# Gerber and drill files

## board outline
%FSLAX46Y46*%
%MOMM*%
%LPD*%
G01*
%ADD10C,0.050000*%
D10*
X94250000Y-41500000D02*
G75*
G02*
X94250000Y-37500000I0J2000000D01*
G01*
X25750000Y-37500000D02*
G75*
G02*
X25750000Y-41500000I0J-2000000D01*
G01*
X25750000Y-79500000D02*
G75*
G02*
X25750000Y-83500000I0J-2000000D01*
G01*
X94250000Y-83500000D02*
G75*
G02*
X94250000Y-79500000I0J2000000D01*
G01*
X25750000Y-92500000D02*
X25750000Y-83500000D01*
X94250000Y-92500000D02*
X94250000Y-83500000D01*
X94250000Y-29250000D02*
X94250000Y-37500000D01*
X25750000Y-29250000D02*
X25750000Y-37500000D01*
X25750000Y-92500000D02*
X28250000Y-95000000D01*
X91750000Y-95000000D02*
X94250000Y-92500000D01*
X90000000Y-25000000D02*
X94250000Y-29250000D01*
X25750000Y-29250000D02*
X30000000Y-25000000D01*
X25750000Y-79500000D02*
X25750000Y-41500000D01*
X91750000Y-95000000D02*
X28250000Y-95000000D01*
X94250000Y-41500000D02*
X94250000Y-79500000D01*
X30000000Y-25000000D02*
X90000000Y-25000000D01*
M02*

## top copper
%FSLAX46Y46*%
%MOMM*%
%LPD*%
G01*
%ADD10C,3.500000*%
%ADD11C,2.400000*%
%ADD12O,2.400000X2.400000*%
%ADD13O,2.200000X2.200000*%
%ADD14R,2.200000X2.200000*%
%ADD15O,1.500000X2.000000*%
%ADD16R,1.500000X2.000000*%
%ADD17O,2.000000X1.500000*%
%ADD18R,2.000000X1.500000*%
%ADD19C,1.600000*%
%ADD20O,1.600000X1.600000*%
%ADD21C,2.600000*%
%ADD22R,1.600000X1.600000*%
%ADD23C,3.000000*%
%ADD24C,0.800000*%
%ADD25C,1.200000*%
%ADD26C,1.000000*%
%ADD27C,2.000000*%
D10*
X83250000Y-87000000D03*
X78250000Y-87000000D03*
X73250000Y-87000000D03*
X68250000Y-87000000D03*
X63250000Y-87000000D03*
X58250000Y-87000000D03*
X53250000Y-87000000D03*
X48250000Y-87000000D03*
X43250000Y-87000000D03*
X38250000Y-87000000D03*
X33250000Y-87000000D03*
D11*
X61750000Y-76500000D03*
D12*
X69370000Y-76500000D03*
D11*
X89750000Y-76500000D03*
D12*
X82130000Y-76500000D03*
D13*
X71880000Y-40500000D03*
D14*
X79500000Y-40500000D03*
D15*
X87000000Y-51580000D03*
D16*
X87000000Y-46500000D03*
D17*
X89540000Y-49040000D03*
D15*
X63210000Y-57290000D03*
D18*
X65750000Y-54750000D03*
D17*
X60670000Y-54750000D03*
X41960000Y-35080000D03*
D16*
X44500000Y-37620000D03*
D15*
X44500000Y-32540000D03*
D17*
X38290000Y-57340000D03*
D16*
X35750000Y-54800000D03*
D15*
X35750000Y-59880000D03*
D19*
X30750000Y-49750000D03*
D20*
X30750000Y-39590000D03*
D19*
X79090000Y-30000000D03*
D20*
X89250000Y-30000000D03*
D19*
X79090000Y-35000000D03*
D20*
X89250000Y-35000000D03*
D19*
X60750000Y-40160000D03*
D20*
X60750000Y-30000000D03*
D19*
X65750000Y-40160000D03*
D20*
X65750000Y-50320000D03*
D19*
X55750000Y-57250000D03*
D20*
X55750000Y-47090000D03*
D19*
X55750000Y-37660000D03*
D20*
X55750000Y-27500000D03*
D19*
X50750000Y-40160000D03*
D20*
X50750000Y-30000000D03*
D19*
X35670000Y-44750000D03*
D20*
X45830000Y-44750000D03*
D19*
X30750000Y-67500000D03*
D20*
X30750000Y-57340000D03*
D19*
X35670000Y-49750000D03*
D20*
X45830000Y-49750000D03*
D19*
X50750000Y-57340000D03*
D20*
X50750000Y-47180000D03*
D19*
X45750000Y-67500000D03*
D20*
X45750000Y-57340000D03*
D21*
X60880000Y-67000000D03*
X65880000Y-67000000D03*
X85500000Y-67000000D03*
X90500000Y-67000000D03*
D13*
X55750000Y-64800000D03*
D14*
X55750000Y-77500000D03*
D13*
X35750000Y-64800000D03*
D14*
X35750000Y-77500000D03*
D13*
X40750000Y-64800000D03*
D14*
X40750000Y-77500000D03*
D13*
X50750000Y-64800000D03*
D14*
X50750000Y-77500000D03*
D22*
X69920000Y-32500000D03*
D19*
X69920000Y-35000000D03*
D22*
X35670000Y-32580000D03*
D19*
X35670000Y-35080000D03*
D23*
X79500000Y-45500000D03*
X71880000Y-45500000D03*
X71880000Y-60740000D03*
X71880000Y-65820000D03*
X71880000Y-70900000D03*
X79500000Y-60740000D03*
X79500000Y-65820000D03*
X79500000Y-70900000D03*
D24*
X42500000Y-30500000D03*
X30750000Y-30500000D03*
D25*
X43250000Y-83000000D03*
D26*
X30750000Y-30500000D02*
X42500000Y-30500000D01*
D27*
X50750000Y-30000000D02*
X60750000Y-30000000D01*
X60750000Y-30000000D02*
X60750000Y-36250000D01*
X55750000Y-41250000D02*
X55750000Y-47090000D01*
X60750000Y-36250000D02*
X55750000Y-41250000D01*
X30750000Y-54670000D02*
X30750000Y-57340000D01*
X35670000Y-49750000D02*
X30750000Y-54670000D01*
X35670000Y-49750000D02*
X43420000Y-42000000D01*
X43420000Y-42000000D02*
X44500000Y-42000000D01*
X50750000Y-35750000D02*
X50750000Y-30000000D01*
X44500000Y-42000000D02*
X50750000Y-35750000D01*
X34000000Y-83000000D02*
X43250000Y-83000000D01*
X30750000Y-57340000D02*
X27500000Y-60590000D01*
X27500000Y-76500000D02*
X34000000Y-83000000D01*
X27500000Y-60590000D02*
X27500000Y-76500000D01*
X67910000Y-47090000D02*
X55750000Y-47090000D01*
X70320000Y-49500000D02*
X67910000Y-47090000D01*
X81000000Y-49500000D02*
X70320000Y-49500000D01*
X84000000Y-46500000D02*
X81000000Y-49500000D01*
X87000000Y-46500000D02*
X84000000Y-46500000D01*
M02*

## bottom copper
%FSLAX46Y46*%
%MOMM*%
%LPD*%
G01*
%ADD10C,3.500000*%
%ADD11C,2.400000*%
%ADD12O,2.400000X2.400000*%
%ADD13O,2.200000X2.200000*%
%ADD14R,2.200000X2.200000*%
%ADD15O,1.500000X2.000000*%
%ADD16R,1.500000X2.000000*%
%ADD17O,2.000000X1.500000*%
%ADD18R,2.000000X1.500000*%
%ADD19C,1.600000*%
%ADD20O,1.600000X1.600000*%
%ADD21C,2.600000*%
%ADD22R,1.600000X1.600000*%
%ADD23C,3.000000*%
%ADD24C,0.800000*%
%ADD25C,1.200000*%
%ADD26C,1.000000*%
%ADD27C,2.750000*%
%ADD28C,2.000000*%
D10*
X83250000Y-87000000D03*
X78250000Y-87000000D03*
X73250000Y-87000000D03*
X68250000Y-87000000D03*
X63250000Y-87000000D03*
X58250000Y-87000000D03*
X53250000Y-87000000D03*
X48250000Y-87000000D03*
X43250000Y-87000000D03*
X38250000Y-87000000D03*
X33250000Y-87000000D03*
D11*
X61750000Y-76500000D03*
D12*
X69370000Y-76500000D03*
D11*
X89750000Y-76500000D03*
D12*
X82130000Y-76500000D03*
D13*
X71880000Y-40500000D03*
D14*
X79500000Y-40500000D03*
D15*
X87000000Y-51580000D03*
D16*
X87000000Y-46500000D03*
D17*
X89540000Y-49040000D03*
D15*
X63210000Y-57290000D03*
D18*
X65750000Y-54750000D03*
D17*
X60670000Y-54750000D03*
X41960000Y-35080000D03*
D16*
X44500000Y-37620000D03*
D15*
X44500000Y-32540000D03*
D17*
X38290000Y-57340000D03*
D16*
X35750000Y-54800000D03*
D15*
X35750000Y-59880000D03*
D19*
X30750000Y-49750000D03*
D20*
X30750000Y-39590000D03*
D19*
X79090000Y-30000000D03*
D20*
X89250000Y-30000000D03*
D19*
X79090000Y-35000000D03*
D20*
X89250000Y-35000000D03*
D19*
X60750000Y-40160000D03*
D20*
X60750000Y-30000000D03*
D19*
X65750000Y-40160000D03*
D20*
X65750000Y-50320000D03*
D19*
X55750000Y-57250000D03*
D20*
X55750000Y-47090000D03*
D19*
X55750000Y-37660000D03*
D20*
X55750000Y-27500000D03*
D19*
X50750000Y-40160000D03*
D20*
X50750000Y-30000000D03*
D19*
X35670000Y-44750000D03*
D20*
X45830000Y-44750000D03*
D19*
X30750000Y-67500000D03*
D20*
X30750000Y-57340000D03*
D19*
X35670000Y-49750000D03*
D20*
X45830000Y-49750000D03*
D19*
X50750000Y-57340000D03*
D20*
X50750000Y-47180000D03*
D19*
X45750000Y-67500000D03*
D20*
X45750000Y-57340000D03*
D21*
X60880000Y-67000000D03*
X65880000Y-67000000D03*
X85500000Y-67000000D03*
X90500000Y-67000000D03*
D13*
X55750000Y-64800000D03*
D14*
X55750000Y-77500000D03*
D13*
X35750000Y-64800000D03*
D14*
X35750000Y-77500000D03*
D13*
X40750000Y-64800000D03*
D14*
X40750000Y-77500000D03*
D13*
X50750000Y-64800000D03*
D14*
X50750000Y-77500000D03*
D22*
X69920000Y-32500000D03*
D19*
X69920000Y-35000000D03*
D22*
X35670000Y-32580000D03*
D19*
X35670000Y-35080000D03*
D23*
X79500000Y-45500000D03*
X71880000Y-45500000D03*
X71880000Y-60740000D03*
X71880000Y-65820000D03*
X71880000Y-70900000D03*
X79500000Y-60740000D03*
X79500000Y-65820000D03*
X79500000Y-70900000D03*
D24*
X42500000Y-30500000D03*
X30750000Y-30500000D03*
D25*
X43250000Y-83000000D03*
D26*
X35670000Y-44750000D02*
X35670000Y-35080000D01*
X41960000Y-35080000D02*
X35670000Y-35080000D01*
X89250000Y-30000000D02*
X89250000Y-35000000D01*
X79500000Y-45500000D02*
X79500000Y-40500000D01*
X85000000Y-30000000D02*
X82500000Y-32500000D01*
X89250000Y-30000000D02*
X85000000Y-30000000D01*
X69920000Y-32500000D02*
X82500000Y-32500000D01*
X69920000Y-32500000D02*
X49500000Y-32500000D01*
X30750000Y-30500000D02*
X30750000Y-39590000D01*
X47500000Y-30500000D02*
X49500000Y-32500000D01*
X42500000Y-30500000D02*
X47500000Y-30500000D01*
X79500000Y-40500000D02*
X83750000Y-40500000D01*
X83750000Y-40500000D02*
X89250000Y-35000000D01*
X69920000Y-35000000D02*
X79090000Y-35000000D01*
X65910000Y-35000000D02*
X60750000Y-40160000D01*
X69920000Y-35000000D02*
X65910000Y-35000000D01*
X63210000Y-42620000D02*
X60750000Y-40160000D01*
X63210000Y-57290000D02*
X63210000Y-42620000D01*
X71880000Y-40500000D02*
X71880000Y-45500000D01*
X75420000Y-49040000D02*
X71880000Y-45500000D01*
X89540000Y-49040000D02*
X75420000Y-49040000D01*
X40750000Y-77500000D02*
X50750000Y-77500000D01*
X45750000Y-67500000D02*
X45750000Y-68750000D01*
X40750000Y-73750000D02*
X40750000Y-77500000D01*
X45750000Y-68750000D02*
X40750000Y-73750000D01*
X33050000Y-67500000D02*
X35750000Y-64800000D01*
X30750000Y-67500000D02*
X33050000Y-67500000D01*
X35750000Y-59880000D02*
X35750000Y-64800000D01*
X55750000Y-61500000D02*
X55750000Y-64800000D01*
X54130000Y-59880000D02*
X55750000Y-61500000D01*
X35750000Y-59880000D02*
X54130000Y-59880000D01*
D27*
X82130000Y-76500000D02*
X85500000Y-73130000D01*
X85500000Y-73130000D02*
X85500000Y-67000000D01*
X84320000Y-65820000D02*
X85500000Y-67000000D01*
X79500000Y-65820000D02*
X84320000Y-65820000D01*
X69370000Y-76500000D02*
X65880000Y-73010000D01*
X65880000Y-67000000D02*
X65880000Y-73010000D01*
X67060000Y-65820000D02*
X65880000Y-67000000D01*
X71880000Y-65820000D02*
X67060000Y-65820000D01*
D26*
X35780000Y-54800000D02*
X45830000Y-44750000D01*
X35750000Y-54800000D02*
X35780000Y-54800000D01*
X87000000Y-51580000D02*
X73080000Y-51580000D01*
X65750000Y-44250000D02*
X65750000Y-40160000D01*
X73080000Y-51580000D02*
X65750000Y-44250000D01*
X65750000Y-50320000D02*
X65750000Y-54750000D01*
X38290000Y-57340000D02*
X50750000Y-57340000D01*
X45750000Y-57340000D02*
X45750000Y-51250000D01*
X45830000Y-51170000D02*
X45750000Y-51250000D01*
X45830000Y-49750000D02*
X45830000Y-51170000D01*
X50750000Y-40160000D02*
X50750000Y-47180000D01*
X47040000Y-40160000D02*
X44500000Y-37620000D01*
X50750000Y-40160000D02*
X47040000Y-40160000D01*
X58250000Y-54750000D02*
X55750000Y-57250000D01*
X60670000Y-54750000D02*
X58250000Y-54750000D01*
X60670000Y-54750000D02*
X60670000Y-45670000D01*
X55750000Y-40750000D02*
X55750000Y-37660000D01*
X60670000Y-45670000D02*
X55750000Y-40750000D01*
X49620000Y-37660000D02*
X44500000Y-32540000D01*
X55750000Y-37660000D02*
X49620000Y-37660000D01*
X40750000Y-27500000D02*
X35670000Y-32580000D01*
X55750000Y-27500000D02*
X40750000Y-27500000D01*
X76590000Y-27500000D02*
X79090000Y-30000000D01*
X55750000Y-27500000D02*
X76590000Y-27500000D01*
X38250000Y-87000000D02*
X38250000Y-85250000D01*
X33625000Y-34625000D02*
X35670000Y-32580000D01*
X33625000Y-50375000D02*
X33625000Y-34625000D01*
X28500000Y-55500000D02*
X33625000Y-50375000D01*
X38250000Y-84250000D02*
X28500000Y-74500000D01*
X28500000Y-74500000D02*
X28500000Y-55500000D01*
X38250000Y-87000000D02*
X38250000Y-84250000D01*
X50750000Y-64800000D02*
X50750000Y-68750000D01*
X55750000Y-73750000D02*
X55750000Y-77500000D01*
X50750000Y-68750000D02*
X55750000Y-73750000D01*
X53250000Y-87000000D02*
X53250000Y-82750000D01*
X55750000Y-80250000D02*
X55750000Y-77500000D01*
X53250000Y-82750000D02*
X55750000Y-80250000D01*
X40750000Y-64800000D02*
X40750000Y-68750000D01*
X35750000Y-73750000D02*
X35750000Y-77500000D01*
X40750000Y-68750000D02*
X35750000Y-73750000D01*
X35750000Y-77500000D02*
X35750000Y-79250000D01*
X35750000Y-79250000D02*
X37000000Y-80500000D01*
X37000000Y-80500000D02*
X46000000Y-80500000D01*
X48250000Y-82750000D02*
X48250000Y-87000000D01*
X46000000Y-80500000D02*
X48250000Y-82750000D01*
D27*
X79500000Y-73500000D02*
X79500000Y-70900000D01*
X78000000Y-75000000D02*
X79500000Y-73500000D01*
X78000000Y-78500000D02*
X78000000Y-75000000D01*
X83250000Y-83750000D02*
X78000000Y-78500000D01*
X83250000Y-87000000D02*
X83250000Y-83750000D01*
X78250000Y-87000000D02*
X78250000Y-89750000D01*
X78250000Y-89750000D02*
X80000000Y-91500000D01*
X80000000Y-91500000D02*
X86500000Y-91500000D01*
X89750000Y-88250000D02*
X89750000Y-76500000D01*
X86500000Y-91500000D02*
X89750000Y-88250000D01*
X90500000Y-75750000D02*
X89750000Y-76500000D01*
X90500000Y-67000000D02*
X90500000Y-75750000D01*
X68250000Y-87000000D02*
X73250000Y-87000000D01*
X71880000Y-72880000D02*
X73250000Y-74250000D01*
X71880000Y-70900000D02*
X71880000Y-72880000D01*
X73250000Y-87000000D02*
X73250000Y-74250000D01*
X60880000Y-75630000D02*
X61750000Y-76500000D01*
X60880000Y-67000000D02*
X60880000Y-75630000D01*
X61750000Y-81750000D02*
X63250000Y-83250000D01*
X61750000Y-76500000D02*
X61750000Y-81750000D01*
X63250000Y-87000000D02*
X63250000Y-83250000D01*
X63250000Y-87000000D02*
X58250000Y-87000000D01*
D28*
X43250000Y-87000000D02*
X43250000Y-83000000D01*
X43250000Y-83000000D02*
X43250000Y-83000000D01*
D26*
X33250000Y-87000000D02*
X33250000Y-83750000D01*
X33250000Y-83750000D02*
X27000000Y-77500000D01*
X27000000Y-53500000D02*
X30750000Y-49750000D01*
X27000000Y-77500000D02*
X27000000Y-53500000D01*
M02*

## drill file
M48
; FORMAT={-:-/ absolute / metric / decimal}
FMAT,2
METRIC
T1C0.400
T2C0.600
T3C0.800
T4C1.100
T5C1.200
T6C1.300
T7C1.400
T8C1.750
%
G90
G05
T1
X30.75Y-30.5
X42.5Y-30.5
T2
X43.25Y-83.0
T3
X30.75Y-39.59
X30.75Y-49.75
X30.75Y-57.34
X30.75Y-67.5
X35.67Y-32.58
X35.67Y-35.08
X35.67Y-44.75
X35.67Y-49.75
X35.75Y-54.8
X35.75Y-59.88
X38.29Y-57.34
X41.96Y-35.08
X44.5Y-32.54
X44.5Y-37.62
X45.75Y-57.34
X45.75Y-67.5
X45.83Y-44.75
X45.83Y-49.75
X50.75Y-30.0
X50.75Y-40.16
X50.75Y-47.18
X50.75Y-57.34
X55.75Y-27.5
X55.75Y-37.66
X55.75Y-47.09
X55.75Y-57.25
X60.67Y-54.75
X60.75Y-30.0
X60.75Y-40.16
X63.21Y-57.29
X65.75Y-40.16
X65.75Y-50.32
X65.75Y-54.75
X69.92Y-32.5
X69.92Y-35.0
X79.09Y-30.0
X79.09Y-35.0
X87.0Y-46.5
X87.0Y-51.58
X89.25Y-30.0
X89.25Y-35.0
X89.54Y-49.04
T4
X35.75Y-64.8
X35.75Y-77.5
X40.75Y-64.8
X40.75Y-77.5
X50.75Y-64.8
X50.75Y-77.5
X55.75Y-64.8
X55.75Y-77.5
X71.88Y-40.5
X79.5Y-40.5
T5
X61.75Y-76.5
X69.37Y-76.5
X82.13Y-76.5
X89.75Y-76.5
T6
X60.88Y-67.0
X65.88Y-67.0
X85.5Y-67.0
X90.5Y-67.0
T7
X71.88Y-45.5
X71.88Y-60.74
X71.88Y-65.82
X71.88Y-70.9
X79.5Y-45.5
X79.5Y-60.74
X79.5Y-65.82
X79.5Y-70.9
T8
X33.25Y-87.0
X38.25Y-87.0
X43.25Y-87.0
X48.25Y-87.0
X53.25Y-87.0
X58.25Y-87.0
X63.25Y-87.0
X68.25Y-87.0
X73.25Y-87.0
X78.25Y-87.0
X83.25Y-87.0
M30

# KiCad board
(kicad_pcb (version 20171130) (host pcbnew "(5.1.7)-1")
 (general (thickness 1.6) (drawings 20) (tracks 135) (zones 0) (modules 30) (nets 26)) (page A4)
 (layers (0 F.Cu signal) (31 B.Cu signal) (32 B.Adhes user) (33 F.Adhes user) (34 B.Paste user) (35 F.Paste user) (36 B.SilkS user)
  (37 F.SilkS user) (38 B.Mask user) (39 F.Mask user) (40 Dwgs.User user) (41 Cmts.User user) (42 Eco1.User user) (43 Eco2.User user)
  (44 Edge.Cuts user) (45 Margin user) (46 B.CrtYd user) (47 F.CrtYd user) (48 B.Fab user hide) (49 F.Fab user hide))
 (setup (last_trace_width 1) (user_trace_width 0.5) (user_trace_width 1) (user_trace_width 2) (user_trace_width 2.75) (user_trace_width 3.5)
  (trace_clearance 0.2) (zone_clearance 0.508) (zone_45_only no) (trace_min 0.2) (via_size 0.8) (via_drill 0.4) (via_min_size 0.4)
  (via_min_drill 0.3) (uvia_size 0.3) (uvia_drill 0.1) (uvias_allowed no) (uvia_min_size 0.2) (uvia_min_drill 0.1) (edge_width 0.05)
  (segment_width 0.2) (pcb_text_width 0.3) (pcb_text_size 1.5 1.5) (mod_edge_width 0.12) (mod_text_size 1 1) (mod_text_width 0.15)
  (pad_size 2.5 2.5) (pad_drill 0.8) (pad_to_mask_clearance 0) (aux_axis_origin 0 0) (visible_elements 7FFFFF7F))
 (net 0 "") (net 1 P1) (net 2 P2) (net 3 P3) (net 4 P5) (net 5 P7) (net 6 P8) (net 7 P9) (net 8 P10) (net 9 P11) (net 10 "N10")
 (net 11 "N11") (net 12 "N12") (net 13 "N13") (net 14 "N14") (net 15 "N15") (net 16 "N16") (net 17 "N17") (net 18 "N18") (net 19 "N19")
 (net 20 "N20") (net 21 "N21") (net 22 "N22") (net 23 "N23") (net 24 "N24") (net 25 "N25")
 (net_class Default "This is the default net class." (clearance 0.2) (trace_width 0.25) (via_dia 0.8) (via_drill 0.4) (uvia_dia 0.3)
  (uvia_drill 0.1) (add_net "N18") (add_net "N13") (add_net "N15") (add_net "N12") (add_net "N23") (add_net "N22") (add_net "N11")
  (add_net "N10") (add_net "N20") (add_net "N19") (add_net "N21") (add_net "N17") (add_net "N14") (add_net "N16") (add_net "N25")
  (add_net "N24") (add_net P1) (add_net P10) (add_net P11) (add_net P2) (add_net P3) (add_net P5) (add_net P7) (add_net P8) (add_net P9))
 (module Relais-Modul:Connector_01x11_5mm (layer F.Cu) (at 83.25 87)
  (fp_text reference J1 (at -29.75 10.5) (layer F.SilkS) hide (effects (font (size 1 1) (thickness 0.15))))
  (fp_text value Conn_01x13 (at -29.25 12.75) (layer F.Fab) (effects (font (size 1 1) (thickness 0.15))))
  (pad 1 thru_hole circle (at 0 0 180) (size 3.5 3.5) (drill 1.75) (layers B.Cu B.Mask) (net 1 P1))
  (pad 2 thru_hole circle (at -5 0 180) (size 3.5 3.5) (drill 1.75) (layers B.Cu B.Mask) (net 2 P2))
  (pad 3 thru_hole circle (at -10 0 180) (size 3.5 3.5) (drill 1.75) (layers B.Cu B.Mask) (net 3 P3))
  (pad 4 thru_hole circle (at -15 0 180) (size 3.5 3.5) (drill 1.75) (layers B.Cu B.Mask) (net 3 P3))
  (pad 5 thru_hole circle (at -20 0 180) (size 3.5 3.5) (drill 1.75) (layers B.Cu B.Mask) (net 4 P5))
  (pad 6 thru_hole circle (at -25 0 180) (size 3.5 3.5) (drill 1.75) (layers B.Cu B.Mask) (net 4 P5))
  (pad 7 thru_hole circle (at -30 0 180) (size 3.5 3.5) (drill 1.75) (layers B.Cu B.Mask) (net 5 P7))
  (pad 8 thru_hole circle (at -35 0 180) (size 3.5 3.5) (drill 1.75) (layers B.Cu B.Mask) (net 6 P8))
  (pad 9 thru_hole circle (at -40 0 180) (size 3.5 3.5) (drill 1.75) (layers B.Cu B.Mask) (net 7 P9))
  (pad 10 thru_hole circle (at -45 0 180) (size 3.5 3.5) (drill 1.75) (layers B.Cu B.Mask) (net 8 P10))
  (pad 11 thru_hole circle (at -50 0 180) (size 3.5 3.5) (drill 1.75) (layers B.Cu B.Mask) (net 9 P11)))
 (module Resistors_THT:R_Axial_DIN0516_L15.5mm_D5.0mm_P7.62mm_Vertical (layer F.Cu) (at 61.75 76.5)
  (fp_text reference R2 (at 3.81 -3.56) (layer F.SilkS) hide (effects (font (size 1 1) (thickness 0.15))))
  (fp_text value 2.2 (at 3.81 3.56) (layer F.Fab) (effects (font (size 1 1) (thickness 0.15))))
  (pad 1 thru_hole circle (at 0 0) (size 2.4 2.4) (drill 1.2) (layers *.Cu *.Mask) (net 4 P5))
  (pad 2 thru_hole oval (at 7.62 0) (size 2.4 2.4) (drill 1.2) (layers *.Cu *.Mask) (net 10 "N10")))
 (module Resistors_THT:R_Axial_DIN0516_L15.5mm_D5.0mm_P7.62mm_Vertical (layer F.Cu) (at 89.75 76.5 180)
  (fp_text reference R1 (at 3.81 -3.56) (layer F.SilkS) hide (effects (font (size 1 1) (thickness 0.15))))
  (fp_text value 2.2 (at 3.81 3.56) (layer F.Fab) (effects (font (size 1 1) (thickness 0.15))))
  (pad 1 thru_hole circle (at 0 0 180) (size 2.4 2.4) (drill 1.2) (layers *.Cu *.Mask) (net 2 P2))
  (pad 2 thru_hole oval (at 7.62 0 180) (size 2.4 2.4) (drill 1.2) (layers *.Cu *.Mask) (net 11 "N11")))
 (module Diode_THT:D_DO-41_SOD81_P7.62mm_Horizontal (layer F.Cu) (at 79.5 40.5 180)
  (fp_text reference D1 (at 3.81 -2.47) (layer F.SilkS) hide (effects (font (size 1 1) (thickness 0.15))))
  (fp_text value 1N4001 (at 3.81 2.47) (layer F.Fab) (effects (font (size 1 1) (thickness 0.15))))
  (pad 2 thru_hole oval (at 7.62 0 180) (size 2.2 2.2) (drill 1.1) (layers *.Cu *.Mask) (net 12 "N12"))
  (pad 1 thru_hole rect (at 0 0 180) (size 2.2 2.2) (drill 1.1) (layers *.Cu *.Mask) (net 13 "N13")))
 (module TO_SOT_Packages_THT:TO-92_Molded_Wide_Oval (layer F.Cu) (at 87 46.5 270)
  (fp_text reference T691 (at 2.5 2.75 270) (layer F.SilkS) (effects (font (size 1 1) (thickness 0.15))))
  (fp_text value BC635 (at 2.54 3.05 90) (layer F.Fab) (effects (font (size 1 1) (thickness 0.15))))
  (pad 3 thru_hole oval (at 5.08 0) (size 1.5 2) (drill 0.8) (layers *.Cu *.Mask) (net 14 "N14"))
  (pad 1 thru_hole rect (at 0 0) (size 1.5 2) (drill 0.8) (layers *.Cu *.Mask) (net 7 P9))
  (pad 2 thru_hole oval (at 2.54 -2.54) (size 2 1.5) (drill 0.8) (layers *.Cu *.Mask) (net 12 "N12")))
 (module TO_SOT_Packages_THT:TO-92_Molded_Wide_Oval (layer F.Cu) (at 65.75 54.75 180)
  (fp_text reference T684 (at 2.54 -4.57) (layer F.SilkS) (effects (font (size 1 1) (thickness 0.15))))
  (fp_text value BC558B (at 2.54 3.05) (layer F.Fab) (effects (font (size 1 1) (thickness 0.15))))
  (pad 2 thru_hole oval (at 2.54 -2.54 270) (size 2 1.5) (drill 0.8) (layers *.Cu *.Mask) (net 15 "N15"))
  (pad 1 thru_hole rect (at 0 0 270) (size 1.5 2) (drill 0.8) (layers *.Cu *.Mask) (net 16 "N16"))
  (pad 3 thru_hole oval (at 5.08 0 270) (size 1.5 2) (drill 0.8) (layers *.Cu *.Mask) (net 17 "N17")))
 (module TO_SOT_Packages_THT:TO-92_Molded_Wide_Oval (layer F.Cu) (at 44.5 37.62 90)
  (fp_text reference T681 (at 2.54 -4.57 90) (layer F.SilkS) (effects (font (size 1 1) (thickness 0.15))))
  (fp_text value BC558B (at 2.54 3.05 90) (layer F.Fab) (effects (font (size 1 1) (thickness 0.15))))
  (pad 2 thru_hole oval (at 2.54 -2.54 180) (size 2 1.5) (drill 0.8) (layers *.Cu *.Mask) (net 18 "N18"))
  (pad 1 thru_hole rect (at 0 0 180) (size 1.5 2) (drill 0.8) (layers *.Cu *.Mask) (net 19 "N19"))
  (pad 3 thru_hole oval (at 5.08 0 180) (size 1.5 2) (drill 0.8) (layers *.Cu *.Mask) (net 17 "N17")))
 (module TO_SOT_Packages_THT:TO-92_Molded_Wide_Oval (layer F.Cu) (at 35.75 54.8 270)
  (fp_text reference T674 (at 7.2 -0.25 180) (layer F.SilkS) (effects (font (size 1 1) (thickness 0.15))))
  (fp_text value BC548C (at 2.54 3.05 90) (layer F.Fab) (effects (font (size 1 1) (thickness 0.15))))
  (pad 2 thru_hole oval (at 2.54 -2.54) (size 2 1.5) (drill 0.8) (layers *.Cu *.Mask) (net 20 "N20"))
  (pad 1 thru_hole rect (at 0 0) (size 1.5 2) (drill 0.8) (layers *.Cu *.Mask) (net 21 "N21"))
  (pad 3 thru_hole oval (at 5.08 0) (size 1.5 2) (drill 0.8) (layers *.Cu *.Mask) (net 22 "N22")))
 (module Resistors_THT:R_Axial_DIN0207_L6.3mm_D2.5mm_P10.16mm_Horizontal (layer F.Cu) (at 30.75 49.75 90)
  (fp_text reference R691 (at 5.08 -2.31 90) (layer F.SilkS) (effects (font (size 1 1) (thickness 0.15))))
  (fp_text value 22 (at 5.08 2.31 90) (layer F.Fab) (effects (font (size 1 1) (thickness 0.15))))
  (pad 1 thru_hole circle (at 0 0 90) (size 1.6 1.6) (drill 0.8) (layers *.Cu *.Mask) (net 9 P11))
  (pad 2 thru_hole oval (at 10.16 0 90) (size 1.6 1.6) (drill 0.8) (layers *.Cu *.Mask) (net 13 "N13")))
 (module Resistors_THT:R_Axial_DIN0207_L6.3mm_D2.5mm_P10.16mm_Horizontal (layer F.Cu) (at 79.09 30)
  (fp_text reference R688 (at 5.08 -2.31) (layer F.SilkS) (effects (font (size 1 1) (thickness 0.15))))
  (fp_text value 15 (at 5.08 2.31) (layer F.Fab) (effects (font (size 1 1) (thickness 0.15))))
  (pad 1 thru_hole circle (at 0 0) (size 1.6 1.6) (drill 0.8) (layers *.Cu *.Mask) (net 8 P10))
  (pad 2 thru_hole oval (at 10.16 0) (size 1.6 1.6) (drill 0.8) (layers *.Cu *.Mask) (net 13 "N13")))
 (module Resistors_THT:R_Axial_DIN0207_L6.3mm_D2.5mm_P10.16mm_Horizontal (layer F.Cu) (at 79.09 35)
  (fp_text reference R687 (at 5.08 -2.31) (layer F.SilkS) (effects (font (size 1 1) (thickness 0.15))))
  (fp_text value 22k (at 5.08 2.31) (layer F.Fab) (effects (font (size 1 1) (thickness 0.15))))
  (pad 1 thru_hole circle (at 0 0) (size 1.6 1.6) (drill 0.8) (layers *.Cu *.Mask) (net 15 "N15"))
  (pad 2 thru_hole oval (at 10.16 0) (size 1.6 1.6) (drill 0.8) (layers *.Cu *.Mask) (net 13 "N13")))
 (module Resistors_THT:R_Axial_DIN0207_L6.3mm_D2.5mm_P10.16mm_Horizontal (layer F.Cu) (at 60.75 40.16 90)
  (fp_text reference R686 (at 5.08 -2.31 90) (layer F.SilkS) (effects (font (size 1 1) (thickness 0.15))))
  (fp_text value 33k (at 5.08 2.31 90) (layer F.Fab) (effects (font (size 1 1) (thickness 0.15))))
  (pad 1 thru_hole circle (at 0 0 90) (size 1.6 1.6) (drill 0.8) (layers *.Cu *.Mask) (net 15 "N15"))
  (pad 2 thru_hole oval (at 10.16 0 90) (size 1.6 1.6) (drill 0.8) (layers *.Cu *.Mask) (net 7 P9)))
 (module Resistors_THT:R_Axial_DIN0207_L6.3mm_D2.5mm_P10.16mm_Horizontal (layer F.Cu) (at 65.75 40.16 270)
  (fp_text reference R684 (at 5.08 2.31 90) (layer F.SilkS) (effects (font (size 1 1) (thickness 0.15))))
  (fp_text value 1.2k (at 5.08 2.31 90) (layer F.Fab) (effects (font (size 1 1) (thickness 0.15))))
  (pad 1 thru_hole circle (at 0 0 270) (size 1.6 1.6) (drill 0.8) (layers *.Cu *.Mask) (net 14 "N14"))
  (pad 2 thru_hole oval (at 10.16 0 270) (size 1.6 1.6) (drill 0.8) (layers *.Cu *.Mask) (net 16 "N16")))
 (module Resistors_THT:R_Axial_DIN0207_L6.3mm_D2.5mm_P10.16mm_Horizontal (layer F.Cu) (at 55.75 57.25 90)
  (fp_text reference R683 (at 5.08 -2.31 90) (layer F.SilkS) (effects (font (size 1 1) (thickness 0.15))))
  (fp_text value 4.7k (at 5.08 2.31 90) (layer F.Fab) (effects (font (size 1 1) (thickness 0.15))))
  (pad 1 thru_hole circle (at 0 0 90) (size 1.6 1.6) (drill 0.8) (layers *.Cu *.Mask) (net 17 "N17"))
  (pad 2 thru_hole oval (at 10.16 0 90) (size 1.6 1.6) (drill 0.8) (layers *.Cu *.Mask) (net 7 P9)))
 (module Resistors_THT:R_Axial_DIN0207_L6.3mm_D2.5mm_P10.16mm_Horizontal (layer F.Cu) (at 55.75 37.66 90)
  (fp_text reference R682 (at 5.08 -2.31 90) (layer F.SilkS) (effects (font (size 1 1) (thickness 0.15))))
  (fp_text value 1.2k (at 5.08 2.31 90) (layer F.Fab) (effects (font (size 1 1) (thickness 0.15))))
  (pad 1 thru_hole circle (at 0 0 90) (size 1.6 1.6) (drill 0.8) (layers *.Cu *.Mask) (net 17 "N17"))
  (pad 2 thru_hole oval (at 10.16 0 90) (size 1.6 1.6) (drill 0.8) (layers *.Cu *.Mask) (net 8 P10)))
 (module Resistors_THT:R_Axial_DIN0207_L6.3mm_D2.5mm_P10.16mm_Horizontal (layer F.Cu) (at 50.75 40.16 90)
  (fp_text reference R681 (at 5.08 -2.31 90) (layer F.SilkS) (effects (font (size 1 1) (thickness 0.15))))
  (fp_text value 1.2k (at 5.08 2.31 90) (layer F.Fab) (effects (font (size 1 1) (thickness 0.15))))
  (pad 1 thru_hole circle (at 0 0 90) (size 1.6 1.6) (drill 0.8) (layers *.Cu *.Mask) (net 19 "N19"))
  (pad 2 thru_hole oval (at 10.16 0 90) (size 1.6 1.6) (drill 0.8) (layers *.Cu *.Mask) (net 7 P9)))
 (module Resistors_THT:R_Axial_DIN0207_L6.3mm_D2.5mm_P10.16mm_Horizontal (layer F.Cu) (at 35.67 44.75)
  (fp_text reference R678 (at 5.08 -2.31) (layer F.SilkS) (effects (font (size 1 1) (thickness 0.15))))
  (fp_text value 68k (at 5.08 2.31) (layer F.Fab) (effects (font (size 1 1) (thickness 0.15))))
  (pad 1 thru_hole circle (at 0 0) (size 1.6 1.6) (drill 0.8) (layers *.Cu *.Mask) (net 18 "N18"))
  (pad 2 thru_hole oval (at 10.16 0) (size 1.6 1.6) (drill 0.8) (layers *.Cu *.Mask) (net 21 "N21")))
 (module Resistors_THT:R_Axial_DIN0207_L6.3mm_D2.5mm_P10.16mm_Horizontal (layer F.Cu) (at 30.75 67.5 90)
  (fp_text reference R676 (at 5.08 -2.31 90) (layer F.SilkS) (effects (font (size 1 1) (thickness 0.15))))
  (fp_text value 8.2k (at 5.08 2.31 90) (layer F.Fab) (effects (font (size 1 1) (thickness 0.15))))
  (pad 1 thru_hole circle (at 0 0 90) (size 1.6 1.6) (drill 0.8) (layers *.Cu *.Mask) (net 22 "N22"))
  (pad 2 thru_hole oval (at 10.16 0 90) (size 1.6 1.6) (drill 0.8) (layers *.Cu *.Mask) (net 7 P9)))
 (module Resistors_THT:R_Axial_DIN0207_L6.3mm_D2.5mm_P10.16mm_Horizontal (layer F.Cu) (at 35.67 49.75)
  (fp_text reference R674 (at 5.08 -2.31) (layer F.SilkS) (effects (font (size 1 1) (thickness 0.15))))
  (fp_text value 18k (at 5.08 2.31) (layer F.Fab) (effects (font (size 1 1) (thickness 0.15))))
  (pad 1 thru_hole circle (at 0 0) (size 1.6 1.6) (drill 0.8) (layers *.Cu *.Mask) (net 7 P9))
  (pad 2 thru_hole oval (at 10.16 0) (size 1.6 1.6) (drill 0.8) (layers *.Cu *.Mask) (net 20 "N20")))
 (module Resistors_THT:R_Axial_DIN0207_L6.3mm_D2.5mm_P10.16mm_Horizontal (layer F.Cu) (at 50.75 57.34 90)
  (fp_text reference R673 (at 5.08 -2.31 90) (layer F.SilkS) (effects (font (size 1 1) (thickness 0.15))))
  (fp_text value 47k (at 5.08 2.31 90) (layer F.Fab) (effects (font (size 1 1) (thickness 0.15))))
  (pad 1 thru_hole circle (at 0 0 90) (size 1.6 1.6) (drill 0.8) (layers *.Cu *.Mask) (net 20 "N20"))
  (pad 2 thru_hole oval (at 10.16 0 90) (size 1.6 1.6) (drill 0.8) (layers *.Cu *.Mask) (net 19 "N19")))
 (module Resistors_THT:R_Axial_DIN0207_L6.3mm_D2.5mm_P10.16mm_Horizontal (layer F.Cu) (at 45.75 67.5 90)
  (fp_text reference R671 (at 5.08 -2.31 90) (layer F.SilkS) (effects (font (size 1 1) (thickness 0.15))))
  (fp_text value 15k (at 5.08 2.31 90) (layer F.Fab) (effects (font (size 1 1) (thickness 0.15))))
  (pad 1 thru_hole circle (at 0 0 90) (size 1.6 1.6) (drill 0.8) (layers *.Cu *.Mask) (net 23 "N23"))
  (pad 2 thru_hole oval (at 10.16 0 90) (size 1.6 1.6) (drill 0.8) (layers *.Cu *.Mask) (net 20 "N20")))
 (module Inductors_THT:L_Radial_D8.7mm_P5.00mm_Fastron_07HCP (layer F.Cu) (at 60.88 67)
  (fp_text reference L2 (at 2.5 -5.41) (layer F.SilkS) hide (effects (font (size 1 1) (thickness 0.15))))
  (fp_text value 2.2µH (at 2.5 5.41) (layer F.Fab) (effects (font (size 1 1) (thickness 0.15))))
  (pad 1 thru_hole circle (at 0 0) (size 2.6 2.6) (drill 1.3) (layers *.Cu *.Mask) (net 4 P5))
  (pad 2 thru_hole circle (at 5 0) (size 2.6 2.6) (drill 1.3) (layers *.Cu *.Mask) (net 10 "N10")))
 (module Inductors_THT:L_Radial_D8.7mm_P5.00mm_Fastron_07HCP (layer F.Cu) (at 85.5 67)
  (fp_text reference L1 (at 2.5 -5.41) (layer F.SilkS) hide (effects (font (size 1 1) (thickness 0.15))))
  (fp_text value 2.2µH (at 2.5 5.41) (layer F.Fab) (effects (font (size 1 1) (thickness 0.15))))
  (pad 1 thru_hole circle (at 0 0) (size 2.6 2.6) (drill 1.3) (layers *.Cu *.Mask) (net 11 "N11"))
  (pad 2 thru_hole circle (at 5 0) (size 2.6 2.6) (drill 1.3) (layers *.Cu *.Mask) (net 2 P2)))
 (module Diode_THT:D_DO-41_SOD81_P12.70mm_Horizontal (layer F.Cu) (at 55.75 77.5 90)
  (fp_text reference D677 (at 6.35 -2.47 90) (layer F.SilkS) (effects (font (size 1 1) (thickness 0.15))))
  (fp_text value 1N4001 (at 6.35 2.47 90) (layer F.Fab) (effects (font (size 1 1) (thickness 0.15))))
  (pad 2 thru_hole oval (at 12.7 0 90) (size 2.2 2.2) (drill 1.1) (layers *.Cu *.Mask) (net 22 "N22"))
  (pad 1 thru_hole rect (at 0 0 90) (size 2.2 2.2) (drill 1.1) (layers *.Cu *.Mask) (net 5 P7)))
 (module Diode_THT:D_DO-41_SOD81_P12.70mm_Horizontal (layer F.Cu) (at 35.75 77.5 90)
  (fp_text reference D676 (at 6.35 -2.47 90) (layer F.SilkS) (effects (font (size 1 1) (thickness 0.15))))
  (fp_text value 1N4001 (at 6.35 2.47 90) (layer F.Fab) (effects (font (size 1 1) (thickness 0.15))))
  (pad 2 thru_hole oval (at 12.7 0 90) (size 2.2 2.2) (drill 1.1) (layers *.Cu *.Mask) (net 22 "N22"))
  (pad 1 thru_hole rect (at 0 0 90) (size 2.2 2.2) (drill 1.1) (layers *.Cu *.Mask) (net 6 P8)))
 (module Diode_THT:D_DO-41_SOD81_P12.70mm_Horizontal (layer F.Cu) (at 40.75 77.5 90)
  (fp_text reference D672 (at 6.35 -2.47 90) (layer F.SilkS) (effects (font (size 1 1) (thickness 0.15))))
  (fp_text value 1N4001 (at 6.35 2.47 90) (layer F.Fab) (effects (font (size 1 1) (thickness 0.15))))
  (pad 2 thru_hole oval (at 12.7 0 90) (size 2.2 2.2) (drill 1.1) (layers *.Cu *.Mask) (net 6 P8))
  (pad 1 thru_hole rect (at 0 0 90) (size 2.2 2.2) (drill 1.1) (layers *.Cu *.Mask) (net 23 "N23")))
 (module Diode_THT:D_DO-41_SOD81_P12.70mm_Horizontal (layer F.Cu) (at 50.75 77.5 90)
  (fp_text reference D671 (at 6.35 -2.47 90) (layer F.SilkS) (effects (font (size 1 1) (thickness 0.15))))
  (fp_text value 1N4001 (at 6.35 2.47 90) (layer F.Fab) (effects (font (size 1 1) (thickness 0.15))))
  (pad 2 thru_hole oval (at 12.7 0 90) (size 2.2 2.2) (drill 1.1) (layers *.Cu *.Mask) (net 5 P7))
  (pad 1 thru_hole rect (at 0 0 90) (size 2.2 2.2) (drill 1.1) (layers *.Cu *.Mask) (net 23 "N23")))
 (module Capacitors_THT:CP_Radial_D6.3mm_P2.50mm (layer F.Cu) (at 69.92 32.5 270)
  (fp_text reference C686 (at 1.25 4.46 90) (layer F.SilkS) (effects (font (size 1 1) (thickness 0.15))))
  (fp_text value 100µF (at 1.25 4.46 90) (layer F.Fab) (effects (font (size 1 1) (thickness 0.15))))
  (pad 1 thru_hole rect (at 0 0 270) (size 1.6 1.6) (drill 0.8) (layers *.Cu *.Mask) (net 13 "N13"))
  (pad 2 thru_hole circle (at 2.5 0 270) (size 1.6 1.6) (drill 0.8) (layers *.Cu *.Mask) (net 15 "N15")))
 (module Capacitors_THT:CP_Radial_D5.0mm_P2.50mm (layer F.Cu) (at 35.67 32.58 270)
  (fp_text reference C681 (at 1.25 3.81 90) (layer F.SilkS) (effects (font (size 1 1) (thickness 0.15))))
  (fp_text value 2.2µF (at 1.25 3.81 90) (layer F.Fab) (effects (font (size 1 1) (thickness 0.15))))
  (pad 1 thru_hole rect (at 0 0 270) (size 1.6 1.6) (drill 0.8) (layers *.Cu *.Mask) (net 8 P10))
  (pad 2 thru_hole circle (at 2.5 0 270) (size 1.6 1.6) (drill 0.8) (layers *.Cu *.Mask) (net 18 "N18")))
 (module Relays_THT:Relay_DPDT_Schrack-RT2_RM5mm (layer F.Cu) (at 79.5 45.5 270)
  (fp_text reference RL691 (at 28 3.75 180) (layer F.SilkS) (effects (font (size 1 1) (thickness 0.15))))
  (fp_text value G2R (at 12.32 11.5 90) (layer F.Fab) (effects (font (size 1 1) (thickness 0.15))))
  (pad A1 thru_hole circle (at 0 0 270) (size 3 3) (drill 1.4) (layers *.Cu *.Mask) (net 13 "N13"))
  (pad A2 thru_hole circle (at 0 7.62 270) (size 3 3) (drill 1.4) (layers *.Cu *.Mask) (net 12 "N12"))
  (pad 22 thru_hole circle (at 15.24 7.62 270) (size 3 3) (drill 1.4) (layers *.Cu *.Mask) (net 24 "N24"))
  (pad 21 thru_hole circle (at 20.32 7.62 270) (size 3 3) (drill 1.4) (layers *.Cu *.Mask) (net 10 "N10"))
  (pad 24 thru_hole circle (at 25.4 7.62 270) (size 3 3) (drill 1.4) (layers *.Cu *.Mask) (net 3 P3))
  (pad 12 thru_hole circle (at 15.24 0 270) (size 3 3) (drill 1.4) (layers *.Cu *.Mask) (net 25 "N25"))
  (pad 11 thru_hole circle (at 20.32 0 270) (size 3 3) (drill 1.4) (layers *.Cu *.Mask) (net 11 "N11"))
  (pad 14 thru_hole circle (at 25.4 0 270) (size 3 3) (drill 1.4) (layers *.Cu *.Mask) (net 1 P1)))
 (gr_arc (start 94.25 39.5) (end 94.25 37.5) (angle -180) (layer Edge.Cuts) (width 0.05))
 (gr_arc (start 25.75 39.5) (end 25.75 41.5) (angle -180) (layer Edge.Cuts) (width 0.05))
 (gr_arc (start 25.75 81.5) (end 25.75 83.5) (angle -180) (layer Edge.Cuts) (width 0.05))
 (gr_arc (start 94.25 81.5) (end 94.25 79.5) (angle -180) (layer Edge.Cuts) (width 0.05))
 (gr_line (start 25.75 92.5) (end 25.75 83.5) (layer Edge.Cuts) (width 0.05))
 (gr_line (start 94.25 92.5) (end 94.25 83.5) (layer Edge.Cuts) (width 0.05))
 (gr_line (start 94.25 29.25) (end 94.25 37.5) (layer Edge.Cuts) (width 0.05))
 (gr_line (start 25.75 29.25) (end 25.75 37.5) (layer Edge.Cuts) (width 0.05))
 (gr_line (start 25.75 92.5) (end 28.25 95) (layer Edge.Cuts) (width 0.05))
 (gr_line (start 91.75 95) (end 94.25 92.5) (layer Edge.Cuts) (width 0.05))
 (gr_line (start 90 25) (end 94.25 29.25) (layer Edge.Cuts) (width 0.05))
 (gr_line (start 25.75 29.25) (end 30 25) (layer Edge.Cuts) (width 0.05))
 (gr_line (start 25.75 79.5) (end 25.75 41.5) (layer Edge.Cuts) (width 0.05))
 (gr_line (start 91.75 95) (end 28.25 95) (layer Edge.Cuts) (width 0.05))
 (gr_line (start 94.25 41.5) (end 94.25 79.5) (layer Edge.Cuts) (width 0.05))
 (gr_line (start 30 25) (end 90 25) (layer Edge.Cuts) (width 0.05))
 (segment (start 35.67 44.75) (end 35.67 35.08) (width 1) (layer B.Cu) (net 18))
 (segment (start 41.96 35.08) (end 35.67 35.08) (width 1) (layer B.Cu) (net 18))
 (segment (start 89.25 30) (end 89.25 35) (width 1) (layer B.Cu) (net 13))
 (segment (start 79.5 45.5) (end 79.5 40.5) (width 1) (layer B.Cu) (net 13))
 (segment (start 85 30) (end 82.5 32.5) (width 1) (layer B.Cu) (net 13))
 (segment (start 89.25 30) (end 85 30) (width 1) (layer B.Cu) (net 13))
 (segment (start 69.92 32.5) (end 82.5 32.5) (width 1) (layer B.Cu) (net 13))
 (segment (start 69.92 32.5) (end 49.5 32.5) (width 1) (layer B.Cu) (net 13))
 (via (at 42.5 30.5) (size 0.8) (drill 0.4) (layers F.Cu B.Cu) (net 13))
 (via (at 30.75 30.5) (size 0.8) (drill 0.4) (layers F.Cu B.Cu) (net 13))
 (segment (start 30.75 30.5) (end 42.5 30.5) (width 1) (layer F.Cu) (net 13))
 (segment (start 30.75 30.5) (end 30.75 39.59) (width 1) (layer B.Cu) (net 13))
 (segment (start 47.5 30.5) (end 49.5 32.5) (width 1) (layer B.Cu) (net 13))
 (segment (start 42.5 30.5) (end 47.5 30.5) (width 1) (layer B.Cu) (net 13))
 (segment (start 79.5 40.5) (end 83.75 40.5) (width 1) (layer B.Cu) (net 13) (status 1000000))
 (segment (start 83.75 40.5) (end 89.25 35) (width 1) (layer B.Cu) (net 13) (status 1000000))
 (segment (start 69.92 35) (end 79.09 35) (width 1) (layer B.Cu) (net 15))
 (segment (start 65.91 35) (end 60.75 40.16) (width 1) (layer B.Cu) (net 15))
 (segment (start 69.92 35) (end 65.91 35) (width 1) (layer B.Cu) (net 15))
 (segment (start 63.21 42.62) (end 60.75 40.16) (width 1) (layer B.Cu) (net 15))
 (segment (start 63.21 57.29) (end 63.21 42.62) (width 1) (layer B.Cu) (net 15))
 (segment (start 71.88 40.5) (end 71.88 45.5) (width 1) (layer B.Cu) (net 12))
 (segment (start 75.42 49.04) (end 71.88 45.5) (width 1) (layer B.Cu) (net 12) (status 1000000))
 (segment (start 89.54 49.04) (end 75.42 49.04) (width 1) (layer B.Cu) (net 12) (status 1000000))
 (segment (start 40.75 77.5) (end 50.75 77.5) (width 1) (layer B.Cu) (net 23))
 (segment (start 45.75 67.5) (end 45.75 68.75) (width 1) (layer B.Cu) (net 23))
 (segment (start 40.75 73.75) (end 40.75 77.5) (width 1) (layer B.Cu) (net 23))
 (segment (start 45.75 68.75) (end 40.75 73.75) (width 1) (layer B.Cu) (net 23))
 (segment (start 33.05 67.5) (end 35.75 64.8) (width 1) (layer B.Cu) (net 22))
 (segment (start 30.75 67.5) (end 33.05 67.5) (width 1) (layer B.Cu) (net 22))
 (segment (start 35.75 59.88) (end 35.75 64.8) (width 1) (layer B.Cu) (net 22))
 (segment (start 55.75 61.5) (end 55.75 64.8) (width 1) (layer B.Cu) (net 22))
 (segment (start 54.13 59.88) (end 55.75 61.5) (width 1) (layer B.Cu) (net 22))
 (segment (start 35.75 59.88) (end 54.13 59.88) (width 1) (layer B.Cu) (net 22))
 (segment (start 82.13 76.5) (end 85.5 73.13) (width 2.75) (layer B.Cu) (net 11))
 (segment (start 85.5 73.13) (end 85.5 67) (width 2.75) (layer B.Cu) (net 11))
 (segment (start 84.32 65.82) (end 85.5 67) (width 2.75) (layer B.Cu) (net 11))
 (segment (start 79.5 65.82) (end 84.32 65.82) (width 2.75) (layer B.Cu) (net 11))
 (segment (start 69.37 76.5) (end 65.88 73.01) (width 2.75) (layer B.Cu) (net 10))
 (segment (start 65.88 67) (end 65.88 73.01) (width 2.75) (layer B.Cu) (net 10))
 (segment (start 67.06 65.82) (end 65.88 67) (width 2.75) (layer B.Cu) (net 10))
 (segment (start 71.88 65.82) (end 67.06 65.82) (width 2.75) (layer B.Cu) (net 10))
 (segment (start 35.78 54.8) (end 45.83 44.75) (width 1) (layer B.Cu) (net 21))
 (segment (start 35.75 54.8) (end 35.78 54.8) (width 1) (layer B.Cu) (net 21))
 (segment (start 87 51.58) (end 73.08 51.58) (width 1) (layer B.Cu) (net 14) (status 1000000))
 (segment (start 65.75 44.25) (end 65.75 40.16) (width 1) (layer B.Cu) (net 14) (status 1000000))
 (segment (start 73.08 51.58) (end 65.75 44.25) (width 1) (layer B.Cu) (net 14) (status 1000000))
 (segment (start 65.75 50.32) (end 65.75 54.75) (width 1) (layer B.Cu) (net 16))
 (segment (start 38.29 57.34) (end 50.75 57.34) (width 1) (layer B.Cu) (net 20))
 (segment (start 45.75 57.34) (end 45.75 51.25) (width 1) (layer B.Cu) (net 20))
 (segment (start 45.83 51.17) (end 45.75 51.25) (width 1) (layer B.Cu) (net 20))
 (segment (start 45.83 49.75) (end 45.83 51.17) (width 1) (layer B.Cu) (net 20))
 (segment (start 50.75 40.16) (end 50.75 47.18) (width 1) (layer B.Cu) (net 19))
 (segment (start 47.04 40.16) (end 44.5 37.62) (width 1) (layer B.Cu) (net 19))
 (segment (start 50.75 40.16) (end 47.04 40.16) (width 1) (layer B.Cu) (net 19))
 (segment (start 58.25 54.75) (end 55.75 57.25) (width 1) (layer B.Cu) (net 17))
 (segment (start 60.67 54.75) (end 58.25 54.75) (width 1) (layer B.Cu) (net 17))
 (segment (start 60.67 54.75) (end 60.67 45.67) (width 1) (layer B.Cu) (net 17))
 (segment (start 55.75 40.75) (end 55.75 37.66) (width 1) (layer B.Cu) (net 17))
 (segment (start 60.67 45.67) (end 55.75 40.75) (width 1) (layer B.Cu) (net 17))
 (segment (start 49.62 37.66) (end 44.5 32.54) (width 1) (layer B.Cu) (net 17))
 (segment (start 55.75 37.66) (end 49.62 37.66) (width 1) (layer B.Cu) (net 17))
 (segment (start 40.75 27.5) (end 35.67 32.58) (width 1) (layer B.Cu) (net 8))
 (segment (start 55.75 27.5) (end 40.75 27.5) (width 1) (layer B.Cu) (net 8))
 (segment (start 76.59 27.5) (end 79.09 30) (width 1) (layer B.Cu) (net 8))
 (segment (start 55.75 27.5) (end 76.59 27.5) (width 1) (layer B.Cu) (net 8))
 (segment (start 38.25 87) (end 38.25 85.25) (width 1) (layer B.Cu) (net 8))
 (segment (start 33.625 34.625) (end 35.67 32.58) (width 1) (layer B.Cu) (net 8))
 (segment (start 33.625 50.375) (end 33.625 34.625) (width 1) (layer B.Cu) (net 8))
 (segment (start 28.5 55.5) (end 33.625 50.375) (width 1) (layer B.Cu) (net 8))
 (segment (start 38.25 84.25) (end 28.5 74.5) (width 1) (layer B.Cu) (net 8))
 (segment (start 28.5 74.5) (end 28.5 55.5) (width 1) (layer B.Cu) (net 8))
 (segment (start 38.25 87) (end 38.25 84.25) (width 1) (layer B.Cu) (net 8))
 (segment (start 50.75 64.8) (end 50.75 68.75) (width 1) (layer B.Cu) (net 5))
 (segment (start 55.75 73.75) (end 55.75 77.5) (width 1) (layer B.Cu) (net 5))
 (segment (start 50.75 68.75) (end 55.75 73.75) (width 1) (layer B.Cu) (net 5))
 (segment (start 53.25 87) (end 53.25 82.75) (width 1) (layer B.Cu) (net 5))
 (segment (start 55.75 80.25) (end 55.75 77.5) (width 1) (layer B.Cu) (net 5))
 (segment (start 53.25 82.75) (end 55.75 80.25) (width 1) (layer B.Cu) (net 5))
 (segment (start 40.75 64.8) (end 40.75 68.75) (width 1) (layer B.Cu) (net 6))
 (segment (start 35.75 73.75) (end 35.75 77.5) (width 1) (layer B.Cu) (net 6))
 (segment (start 40.75 68.75) (end 35.75 73.75) (width 1) (layer B.Cu) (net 6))
 (segment (start 35.75 77.5) (end 35.75 79.25) (width 1) (layer B.Cu) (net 6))
 (segment (start 35.75 79.25) (end 37 80.5) (width 1) (layer B.Cu) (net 6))
 (segment (start 37 80.5) (end 46 80.5) (width 1) (layer B.Cu) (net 6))
 (segment (start 48.25 82.75) (end 48.25 87) (width 1) (layer B.Cu) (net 6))
 (segment (start 46 80.5) (end 48.25 82.75) (width 1) (layer B.Cu) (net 6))
 (segment (start 79.5 73.5) (end 79.5 70.9) (width 2.75) (layer B.Cu) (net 1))
 (segment (start 78 75) (end 79.5 73.5) (width 2.75) (layer B.Cu) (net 1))
 (segment (start 78 78.5) (end 78 75) (width 2.75) (layer B.Cu) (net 1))
 (segment (start 83.25 83.75) (end 78 78.5) (width 2.75) (layer B.Cu) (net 1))
 (segment (start 83.25 87) (end 83.25 83.75) (width 2.75) (layer B.Cu) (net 1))
 (segment (start 78.25 87) (end 78.25 89.75) (width 2.75) (layer B.Cu) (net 2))
 (segment (start 78.25 89.75) (end 80 91.5) (width 2.75) (layer B.Cu) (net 2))
 (segment (start 80 91.5) (end 86.5 91.5) (width 2.75) (layer B.Cu) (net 2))
 (segment (start 89.75 88.25) (end 89.75 76.5) (width 2.75) (layer B.Cu) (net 2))
 (segment (start 86.5 91.5) (end 89.75 88.25) (width 2.75) (layer B.Cu) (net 2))
 (segment (start 90.5 75.75) (end 89.75 76.5) (width 2.75) (layer B.Cu) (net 2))
 (segment (start 90.5 67) (end 90.5 75.75) (width 2.75) (layer B.Cu) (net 2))
 (segment (start 68.25 87) (end 73.25 87) (width 2.75) (layer B.Cu) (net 3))
 (segment (start 71.88 72.88) (end 73.25 74.25) (width 2.75) (layer B.Cu) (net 3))
 (segment (start 71.88 70.9) (end 71.88 72.88) (width 2.75) (layer B.Cu) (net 3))
 (segment (start 73.25 87) (end 73.25 74.25) (width 2.75) (layer B.Cu) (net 3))
 (segment (start 60.88 75.63) (end 61.75 76.5) (width 2.75) (layer B.Cu) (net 4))
 (segment (start 60.88 67) (end 60.88 75.63) (width 2.75) (layer B.Cu) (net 4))
 (segment (start 61.75 81.75) (end 63.25 83.25) (width 2.75) (layer B.Cu) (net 4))
 (segment (start 61.75 76.5) (end 61.75 81.75) (width 2.75) (layer B.Cu) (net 4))
 (segment (start 63.25 87) (end 63.25 83.25) (width 2.75) (layer B.Cu) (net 4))
 (segment (start 63.25 87) (end 58.25 87) (width 2.75) (layer B.Cu) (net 4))
 (segment (start 50.75 30) (end 60.75 30) (width 2) (layer F.Cu) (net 7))
 (segment (start 60.75 30) (end 60.75 36.25) (width 2) (layer F.Cu) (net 7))
 (segment (start 55.75 41.25) (end 55.75 47.09) (width 2) (layer F.Cu) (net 7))
 (segment (start 60.75 36.25) (end 55.75 41.25) (width 2) (layer F.Cu) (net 7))
 (segment (start 30.75 54.67) (end 30.75 57.34) (width 2) (layer F.Cu) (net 7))
 (segment (start 35.67 49.75) (end 30.75 54.67) (width 2) (layer F.Cu) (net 7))
 (segment (start 35.67 49.75) (end 43.42 42) (width 2) (layer F.Cu) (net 7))
 (segment (start 43.42 42) (end 44.5 42) (width 2) (layer F.Cu) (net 7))
 (segment (start 50.75 35.75) (end 50.75 30) (width 2) (layer F.Cu) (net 7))
 (segment (start 44.5 42) (end 50.75 35.75) (width 2) (layer F.Cu) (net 7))
 (segment (start 43.25 87) (end 43.25 83) (width 2) (layer B.Cu) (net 7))
 (segment (start 43.25 83) (end 43.25 83) (width 2) (layer B.Cu) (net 7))
 (via (at 43.25 83) (size 1.2) (drill 0.6) (layers F.Cu B.Cu) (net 7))
 (segment (start 34 83) (end 43.25 83) (width 2) (layer F.Cu) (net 7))
 (segment (start 30.75 57.34) (end 27.5 60.59) (width 2) (layer F.Cu) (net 7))
 (segment (start 27.5 76.5) (end 34 83) (width 2) (layer F.Cu) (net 7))
 (segment (start 27.5 60.59) (end 27.5 76.5) (width 2) (layer F.Cu) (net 7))
 (segment (start 67.91 47.09) (end 55.75 47.09) (width 2) (layer F.Cu) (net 7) (status 1000000))
 (segment (start 70.32 49.5) (end 67.91 47.09) (width 2) (layer F.Cu) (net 7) (status 1000000))
 (segment (start 81 49.5) (end 70.32 49.5) (width 2) (layer F.Cu) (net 7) (status 1000000))
 (segment (start 84 46.5) (end 81 49.5) (width 2) (layer F.Cu) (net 7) (status 1000000))
 (segment (start 87 46.5) (end 84 46.5) (width 2) (layer F.Cu) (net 7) (status 1000000))
 (segment (start 33.25 87) (end 33.25 83.75) (width 1) (layer B.Cu) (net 9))
 (segment (start 33.25 83.75) (end 27 77.5) (width 1) (layer B.Cu) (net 9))
 (segment (start 27 53.5) (end 30.75 49.75) (width 1) (layer B.Cu) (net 9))
 (segment (start 27 77.5) (end 27 53.5) (width 1) (layer B.Cu) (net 9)))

